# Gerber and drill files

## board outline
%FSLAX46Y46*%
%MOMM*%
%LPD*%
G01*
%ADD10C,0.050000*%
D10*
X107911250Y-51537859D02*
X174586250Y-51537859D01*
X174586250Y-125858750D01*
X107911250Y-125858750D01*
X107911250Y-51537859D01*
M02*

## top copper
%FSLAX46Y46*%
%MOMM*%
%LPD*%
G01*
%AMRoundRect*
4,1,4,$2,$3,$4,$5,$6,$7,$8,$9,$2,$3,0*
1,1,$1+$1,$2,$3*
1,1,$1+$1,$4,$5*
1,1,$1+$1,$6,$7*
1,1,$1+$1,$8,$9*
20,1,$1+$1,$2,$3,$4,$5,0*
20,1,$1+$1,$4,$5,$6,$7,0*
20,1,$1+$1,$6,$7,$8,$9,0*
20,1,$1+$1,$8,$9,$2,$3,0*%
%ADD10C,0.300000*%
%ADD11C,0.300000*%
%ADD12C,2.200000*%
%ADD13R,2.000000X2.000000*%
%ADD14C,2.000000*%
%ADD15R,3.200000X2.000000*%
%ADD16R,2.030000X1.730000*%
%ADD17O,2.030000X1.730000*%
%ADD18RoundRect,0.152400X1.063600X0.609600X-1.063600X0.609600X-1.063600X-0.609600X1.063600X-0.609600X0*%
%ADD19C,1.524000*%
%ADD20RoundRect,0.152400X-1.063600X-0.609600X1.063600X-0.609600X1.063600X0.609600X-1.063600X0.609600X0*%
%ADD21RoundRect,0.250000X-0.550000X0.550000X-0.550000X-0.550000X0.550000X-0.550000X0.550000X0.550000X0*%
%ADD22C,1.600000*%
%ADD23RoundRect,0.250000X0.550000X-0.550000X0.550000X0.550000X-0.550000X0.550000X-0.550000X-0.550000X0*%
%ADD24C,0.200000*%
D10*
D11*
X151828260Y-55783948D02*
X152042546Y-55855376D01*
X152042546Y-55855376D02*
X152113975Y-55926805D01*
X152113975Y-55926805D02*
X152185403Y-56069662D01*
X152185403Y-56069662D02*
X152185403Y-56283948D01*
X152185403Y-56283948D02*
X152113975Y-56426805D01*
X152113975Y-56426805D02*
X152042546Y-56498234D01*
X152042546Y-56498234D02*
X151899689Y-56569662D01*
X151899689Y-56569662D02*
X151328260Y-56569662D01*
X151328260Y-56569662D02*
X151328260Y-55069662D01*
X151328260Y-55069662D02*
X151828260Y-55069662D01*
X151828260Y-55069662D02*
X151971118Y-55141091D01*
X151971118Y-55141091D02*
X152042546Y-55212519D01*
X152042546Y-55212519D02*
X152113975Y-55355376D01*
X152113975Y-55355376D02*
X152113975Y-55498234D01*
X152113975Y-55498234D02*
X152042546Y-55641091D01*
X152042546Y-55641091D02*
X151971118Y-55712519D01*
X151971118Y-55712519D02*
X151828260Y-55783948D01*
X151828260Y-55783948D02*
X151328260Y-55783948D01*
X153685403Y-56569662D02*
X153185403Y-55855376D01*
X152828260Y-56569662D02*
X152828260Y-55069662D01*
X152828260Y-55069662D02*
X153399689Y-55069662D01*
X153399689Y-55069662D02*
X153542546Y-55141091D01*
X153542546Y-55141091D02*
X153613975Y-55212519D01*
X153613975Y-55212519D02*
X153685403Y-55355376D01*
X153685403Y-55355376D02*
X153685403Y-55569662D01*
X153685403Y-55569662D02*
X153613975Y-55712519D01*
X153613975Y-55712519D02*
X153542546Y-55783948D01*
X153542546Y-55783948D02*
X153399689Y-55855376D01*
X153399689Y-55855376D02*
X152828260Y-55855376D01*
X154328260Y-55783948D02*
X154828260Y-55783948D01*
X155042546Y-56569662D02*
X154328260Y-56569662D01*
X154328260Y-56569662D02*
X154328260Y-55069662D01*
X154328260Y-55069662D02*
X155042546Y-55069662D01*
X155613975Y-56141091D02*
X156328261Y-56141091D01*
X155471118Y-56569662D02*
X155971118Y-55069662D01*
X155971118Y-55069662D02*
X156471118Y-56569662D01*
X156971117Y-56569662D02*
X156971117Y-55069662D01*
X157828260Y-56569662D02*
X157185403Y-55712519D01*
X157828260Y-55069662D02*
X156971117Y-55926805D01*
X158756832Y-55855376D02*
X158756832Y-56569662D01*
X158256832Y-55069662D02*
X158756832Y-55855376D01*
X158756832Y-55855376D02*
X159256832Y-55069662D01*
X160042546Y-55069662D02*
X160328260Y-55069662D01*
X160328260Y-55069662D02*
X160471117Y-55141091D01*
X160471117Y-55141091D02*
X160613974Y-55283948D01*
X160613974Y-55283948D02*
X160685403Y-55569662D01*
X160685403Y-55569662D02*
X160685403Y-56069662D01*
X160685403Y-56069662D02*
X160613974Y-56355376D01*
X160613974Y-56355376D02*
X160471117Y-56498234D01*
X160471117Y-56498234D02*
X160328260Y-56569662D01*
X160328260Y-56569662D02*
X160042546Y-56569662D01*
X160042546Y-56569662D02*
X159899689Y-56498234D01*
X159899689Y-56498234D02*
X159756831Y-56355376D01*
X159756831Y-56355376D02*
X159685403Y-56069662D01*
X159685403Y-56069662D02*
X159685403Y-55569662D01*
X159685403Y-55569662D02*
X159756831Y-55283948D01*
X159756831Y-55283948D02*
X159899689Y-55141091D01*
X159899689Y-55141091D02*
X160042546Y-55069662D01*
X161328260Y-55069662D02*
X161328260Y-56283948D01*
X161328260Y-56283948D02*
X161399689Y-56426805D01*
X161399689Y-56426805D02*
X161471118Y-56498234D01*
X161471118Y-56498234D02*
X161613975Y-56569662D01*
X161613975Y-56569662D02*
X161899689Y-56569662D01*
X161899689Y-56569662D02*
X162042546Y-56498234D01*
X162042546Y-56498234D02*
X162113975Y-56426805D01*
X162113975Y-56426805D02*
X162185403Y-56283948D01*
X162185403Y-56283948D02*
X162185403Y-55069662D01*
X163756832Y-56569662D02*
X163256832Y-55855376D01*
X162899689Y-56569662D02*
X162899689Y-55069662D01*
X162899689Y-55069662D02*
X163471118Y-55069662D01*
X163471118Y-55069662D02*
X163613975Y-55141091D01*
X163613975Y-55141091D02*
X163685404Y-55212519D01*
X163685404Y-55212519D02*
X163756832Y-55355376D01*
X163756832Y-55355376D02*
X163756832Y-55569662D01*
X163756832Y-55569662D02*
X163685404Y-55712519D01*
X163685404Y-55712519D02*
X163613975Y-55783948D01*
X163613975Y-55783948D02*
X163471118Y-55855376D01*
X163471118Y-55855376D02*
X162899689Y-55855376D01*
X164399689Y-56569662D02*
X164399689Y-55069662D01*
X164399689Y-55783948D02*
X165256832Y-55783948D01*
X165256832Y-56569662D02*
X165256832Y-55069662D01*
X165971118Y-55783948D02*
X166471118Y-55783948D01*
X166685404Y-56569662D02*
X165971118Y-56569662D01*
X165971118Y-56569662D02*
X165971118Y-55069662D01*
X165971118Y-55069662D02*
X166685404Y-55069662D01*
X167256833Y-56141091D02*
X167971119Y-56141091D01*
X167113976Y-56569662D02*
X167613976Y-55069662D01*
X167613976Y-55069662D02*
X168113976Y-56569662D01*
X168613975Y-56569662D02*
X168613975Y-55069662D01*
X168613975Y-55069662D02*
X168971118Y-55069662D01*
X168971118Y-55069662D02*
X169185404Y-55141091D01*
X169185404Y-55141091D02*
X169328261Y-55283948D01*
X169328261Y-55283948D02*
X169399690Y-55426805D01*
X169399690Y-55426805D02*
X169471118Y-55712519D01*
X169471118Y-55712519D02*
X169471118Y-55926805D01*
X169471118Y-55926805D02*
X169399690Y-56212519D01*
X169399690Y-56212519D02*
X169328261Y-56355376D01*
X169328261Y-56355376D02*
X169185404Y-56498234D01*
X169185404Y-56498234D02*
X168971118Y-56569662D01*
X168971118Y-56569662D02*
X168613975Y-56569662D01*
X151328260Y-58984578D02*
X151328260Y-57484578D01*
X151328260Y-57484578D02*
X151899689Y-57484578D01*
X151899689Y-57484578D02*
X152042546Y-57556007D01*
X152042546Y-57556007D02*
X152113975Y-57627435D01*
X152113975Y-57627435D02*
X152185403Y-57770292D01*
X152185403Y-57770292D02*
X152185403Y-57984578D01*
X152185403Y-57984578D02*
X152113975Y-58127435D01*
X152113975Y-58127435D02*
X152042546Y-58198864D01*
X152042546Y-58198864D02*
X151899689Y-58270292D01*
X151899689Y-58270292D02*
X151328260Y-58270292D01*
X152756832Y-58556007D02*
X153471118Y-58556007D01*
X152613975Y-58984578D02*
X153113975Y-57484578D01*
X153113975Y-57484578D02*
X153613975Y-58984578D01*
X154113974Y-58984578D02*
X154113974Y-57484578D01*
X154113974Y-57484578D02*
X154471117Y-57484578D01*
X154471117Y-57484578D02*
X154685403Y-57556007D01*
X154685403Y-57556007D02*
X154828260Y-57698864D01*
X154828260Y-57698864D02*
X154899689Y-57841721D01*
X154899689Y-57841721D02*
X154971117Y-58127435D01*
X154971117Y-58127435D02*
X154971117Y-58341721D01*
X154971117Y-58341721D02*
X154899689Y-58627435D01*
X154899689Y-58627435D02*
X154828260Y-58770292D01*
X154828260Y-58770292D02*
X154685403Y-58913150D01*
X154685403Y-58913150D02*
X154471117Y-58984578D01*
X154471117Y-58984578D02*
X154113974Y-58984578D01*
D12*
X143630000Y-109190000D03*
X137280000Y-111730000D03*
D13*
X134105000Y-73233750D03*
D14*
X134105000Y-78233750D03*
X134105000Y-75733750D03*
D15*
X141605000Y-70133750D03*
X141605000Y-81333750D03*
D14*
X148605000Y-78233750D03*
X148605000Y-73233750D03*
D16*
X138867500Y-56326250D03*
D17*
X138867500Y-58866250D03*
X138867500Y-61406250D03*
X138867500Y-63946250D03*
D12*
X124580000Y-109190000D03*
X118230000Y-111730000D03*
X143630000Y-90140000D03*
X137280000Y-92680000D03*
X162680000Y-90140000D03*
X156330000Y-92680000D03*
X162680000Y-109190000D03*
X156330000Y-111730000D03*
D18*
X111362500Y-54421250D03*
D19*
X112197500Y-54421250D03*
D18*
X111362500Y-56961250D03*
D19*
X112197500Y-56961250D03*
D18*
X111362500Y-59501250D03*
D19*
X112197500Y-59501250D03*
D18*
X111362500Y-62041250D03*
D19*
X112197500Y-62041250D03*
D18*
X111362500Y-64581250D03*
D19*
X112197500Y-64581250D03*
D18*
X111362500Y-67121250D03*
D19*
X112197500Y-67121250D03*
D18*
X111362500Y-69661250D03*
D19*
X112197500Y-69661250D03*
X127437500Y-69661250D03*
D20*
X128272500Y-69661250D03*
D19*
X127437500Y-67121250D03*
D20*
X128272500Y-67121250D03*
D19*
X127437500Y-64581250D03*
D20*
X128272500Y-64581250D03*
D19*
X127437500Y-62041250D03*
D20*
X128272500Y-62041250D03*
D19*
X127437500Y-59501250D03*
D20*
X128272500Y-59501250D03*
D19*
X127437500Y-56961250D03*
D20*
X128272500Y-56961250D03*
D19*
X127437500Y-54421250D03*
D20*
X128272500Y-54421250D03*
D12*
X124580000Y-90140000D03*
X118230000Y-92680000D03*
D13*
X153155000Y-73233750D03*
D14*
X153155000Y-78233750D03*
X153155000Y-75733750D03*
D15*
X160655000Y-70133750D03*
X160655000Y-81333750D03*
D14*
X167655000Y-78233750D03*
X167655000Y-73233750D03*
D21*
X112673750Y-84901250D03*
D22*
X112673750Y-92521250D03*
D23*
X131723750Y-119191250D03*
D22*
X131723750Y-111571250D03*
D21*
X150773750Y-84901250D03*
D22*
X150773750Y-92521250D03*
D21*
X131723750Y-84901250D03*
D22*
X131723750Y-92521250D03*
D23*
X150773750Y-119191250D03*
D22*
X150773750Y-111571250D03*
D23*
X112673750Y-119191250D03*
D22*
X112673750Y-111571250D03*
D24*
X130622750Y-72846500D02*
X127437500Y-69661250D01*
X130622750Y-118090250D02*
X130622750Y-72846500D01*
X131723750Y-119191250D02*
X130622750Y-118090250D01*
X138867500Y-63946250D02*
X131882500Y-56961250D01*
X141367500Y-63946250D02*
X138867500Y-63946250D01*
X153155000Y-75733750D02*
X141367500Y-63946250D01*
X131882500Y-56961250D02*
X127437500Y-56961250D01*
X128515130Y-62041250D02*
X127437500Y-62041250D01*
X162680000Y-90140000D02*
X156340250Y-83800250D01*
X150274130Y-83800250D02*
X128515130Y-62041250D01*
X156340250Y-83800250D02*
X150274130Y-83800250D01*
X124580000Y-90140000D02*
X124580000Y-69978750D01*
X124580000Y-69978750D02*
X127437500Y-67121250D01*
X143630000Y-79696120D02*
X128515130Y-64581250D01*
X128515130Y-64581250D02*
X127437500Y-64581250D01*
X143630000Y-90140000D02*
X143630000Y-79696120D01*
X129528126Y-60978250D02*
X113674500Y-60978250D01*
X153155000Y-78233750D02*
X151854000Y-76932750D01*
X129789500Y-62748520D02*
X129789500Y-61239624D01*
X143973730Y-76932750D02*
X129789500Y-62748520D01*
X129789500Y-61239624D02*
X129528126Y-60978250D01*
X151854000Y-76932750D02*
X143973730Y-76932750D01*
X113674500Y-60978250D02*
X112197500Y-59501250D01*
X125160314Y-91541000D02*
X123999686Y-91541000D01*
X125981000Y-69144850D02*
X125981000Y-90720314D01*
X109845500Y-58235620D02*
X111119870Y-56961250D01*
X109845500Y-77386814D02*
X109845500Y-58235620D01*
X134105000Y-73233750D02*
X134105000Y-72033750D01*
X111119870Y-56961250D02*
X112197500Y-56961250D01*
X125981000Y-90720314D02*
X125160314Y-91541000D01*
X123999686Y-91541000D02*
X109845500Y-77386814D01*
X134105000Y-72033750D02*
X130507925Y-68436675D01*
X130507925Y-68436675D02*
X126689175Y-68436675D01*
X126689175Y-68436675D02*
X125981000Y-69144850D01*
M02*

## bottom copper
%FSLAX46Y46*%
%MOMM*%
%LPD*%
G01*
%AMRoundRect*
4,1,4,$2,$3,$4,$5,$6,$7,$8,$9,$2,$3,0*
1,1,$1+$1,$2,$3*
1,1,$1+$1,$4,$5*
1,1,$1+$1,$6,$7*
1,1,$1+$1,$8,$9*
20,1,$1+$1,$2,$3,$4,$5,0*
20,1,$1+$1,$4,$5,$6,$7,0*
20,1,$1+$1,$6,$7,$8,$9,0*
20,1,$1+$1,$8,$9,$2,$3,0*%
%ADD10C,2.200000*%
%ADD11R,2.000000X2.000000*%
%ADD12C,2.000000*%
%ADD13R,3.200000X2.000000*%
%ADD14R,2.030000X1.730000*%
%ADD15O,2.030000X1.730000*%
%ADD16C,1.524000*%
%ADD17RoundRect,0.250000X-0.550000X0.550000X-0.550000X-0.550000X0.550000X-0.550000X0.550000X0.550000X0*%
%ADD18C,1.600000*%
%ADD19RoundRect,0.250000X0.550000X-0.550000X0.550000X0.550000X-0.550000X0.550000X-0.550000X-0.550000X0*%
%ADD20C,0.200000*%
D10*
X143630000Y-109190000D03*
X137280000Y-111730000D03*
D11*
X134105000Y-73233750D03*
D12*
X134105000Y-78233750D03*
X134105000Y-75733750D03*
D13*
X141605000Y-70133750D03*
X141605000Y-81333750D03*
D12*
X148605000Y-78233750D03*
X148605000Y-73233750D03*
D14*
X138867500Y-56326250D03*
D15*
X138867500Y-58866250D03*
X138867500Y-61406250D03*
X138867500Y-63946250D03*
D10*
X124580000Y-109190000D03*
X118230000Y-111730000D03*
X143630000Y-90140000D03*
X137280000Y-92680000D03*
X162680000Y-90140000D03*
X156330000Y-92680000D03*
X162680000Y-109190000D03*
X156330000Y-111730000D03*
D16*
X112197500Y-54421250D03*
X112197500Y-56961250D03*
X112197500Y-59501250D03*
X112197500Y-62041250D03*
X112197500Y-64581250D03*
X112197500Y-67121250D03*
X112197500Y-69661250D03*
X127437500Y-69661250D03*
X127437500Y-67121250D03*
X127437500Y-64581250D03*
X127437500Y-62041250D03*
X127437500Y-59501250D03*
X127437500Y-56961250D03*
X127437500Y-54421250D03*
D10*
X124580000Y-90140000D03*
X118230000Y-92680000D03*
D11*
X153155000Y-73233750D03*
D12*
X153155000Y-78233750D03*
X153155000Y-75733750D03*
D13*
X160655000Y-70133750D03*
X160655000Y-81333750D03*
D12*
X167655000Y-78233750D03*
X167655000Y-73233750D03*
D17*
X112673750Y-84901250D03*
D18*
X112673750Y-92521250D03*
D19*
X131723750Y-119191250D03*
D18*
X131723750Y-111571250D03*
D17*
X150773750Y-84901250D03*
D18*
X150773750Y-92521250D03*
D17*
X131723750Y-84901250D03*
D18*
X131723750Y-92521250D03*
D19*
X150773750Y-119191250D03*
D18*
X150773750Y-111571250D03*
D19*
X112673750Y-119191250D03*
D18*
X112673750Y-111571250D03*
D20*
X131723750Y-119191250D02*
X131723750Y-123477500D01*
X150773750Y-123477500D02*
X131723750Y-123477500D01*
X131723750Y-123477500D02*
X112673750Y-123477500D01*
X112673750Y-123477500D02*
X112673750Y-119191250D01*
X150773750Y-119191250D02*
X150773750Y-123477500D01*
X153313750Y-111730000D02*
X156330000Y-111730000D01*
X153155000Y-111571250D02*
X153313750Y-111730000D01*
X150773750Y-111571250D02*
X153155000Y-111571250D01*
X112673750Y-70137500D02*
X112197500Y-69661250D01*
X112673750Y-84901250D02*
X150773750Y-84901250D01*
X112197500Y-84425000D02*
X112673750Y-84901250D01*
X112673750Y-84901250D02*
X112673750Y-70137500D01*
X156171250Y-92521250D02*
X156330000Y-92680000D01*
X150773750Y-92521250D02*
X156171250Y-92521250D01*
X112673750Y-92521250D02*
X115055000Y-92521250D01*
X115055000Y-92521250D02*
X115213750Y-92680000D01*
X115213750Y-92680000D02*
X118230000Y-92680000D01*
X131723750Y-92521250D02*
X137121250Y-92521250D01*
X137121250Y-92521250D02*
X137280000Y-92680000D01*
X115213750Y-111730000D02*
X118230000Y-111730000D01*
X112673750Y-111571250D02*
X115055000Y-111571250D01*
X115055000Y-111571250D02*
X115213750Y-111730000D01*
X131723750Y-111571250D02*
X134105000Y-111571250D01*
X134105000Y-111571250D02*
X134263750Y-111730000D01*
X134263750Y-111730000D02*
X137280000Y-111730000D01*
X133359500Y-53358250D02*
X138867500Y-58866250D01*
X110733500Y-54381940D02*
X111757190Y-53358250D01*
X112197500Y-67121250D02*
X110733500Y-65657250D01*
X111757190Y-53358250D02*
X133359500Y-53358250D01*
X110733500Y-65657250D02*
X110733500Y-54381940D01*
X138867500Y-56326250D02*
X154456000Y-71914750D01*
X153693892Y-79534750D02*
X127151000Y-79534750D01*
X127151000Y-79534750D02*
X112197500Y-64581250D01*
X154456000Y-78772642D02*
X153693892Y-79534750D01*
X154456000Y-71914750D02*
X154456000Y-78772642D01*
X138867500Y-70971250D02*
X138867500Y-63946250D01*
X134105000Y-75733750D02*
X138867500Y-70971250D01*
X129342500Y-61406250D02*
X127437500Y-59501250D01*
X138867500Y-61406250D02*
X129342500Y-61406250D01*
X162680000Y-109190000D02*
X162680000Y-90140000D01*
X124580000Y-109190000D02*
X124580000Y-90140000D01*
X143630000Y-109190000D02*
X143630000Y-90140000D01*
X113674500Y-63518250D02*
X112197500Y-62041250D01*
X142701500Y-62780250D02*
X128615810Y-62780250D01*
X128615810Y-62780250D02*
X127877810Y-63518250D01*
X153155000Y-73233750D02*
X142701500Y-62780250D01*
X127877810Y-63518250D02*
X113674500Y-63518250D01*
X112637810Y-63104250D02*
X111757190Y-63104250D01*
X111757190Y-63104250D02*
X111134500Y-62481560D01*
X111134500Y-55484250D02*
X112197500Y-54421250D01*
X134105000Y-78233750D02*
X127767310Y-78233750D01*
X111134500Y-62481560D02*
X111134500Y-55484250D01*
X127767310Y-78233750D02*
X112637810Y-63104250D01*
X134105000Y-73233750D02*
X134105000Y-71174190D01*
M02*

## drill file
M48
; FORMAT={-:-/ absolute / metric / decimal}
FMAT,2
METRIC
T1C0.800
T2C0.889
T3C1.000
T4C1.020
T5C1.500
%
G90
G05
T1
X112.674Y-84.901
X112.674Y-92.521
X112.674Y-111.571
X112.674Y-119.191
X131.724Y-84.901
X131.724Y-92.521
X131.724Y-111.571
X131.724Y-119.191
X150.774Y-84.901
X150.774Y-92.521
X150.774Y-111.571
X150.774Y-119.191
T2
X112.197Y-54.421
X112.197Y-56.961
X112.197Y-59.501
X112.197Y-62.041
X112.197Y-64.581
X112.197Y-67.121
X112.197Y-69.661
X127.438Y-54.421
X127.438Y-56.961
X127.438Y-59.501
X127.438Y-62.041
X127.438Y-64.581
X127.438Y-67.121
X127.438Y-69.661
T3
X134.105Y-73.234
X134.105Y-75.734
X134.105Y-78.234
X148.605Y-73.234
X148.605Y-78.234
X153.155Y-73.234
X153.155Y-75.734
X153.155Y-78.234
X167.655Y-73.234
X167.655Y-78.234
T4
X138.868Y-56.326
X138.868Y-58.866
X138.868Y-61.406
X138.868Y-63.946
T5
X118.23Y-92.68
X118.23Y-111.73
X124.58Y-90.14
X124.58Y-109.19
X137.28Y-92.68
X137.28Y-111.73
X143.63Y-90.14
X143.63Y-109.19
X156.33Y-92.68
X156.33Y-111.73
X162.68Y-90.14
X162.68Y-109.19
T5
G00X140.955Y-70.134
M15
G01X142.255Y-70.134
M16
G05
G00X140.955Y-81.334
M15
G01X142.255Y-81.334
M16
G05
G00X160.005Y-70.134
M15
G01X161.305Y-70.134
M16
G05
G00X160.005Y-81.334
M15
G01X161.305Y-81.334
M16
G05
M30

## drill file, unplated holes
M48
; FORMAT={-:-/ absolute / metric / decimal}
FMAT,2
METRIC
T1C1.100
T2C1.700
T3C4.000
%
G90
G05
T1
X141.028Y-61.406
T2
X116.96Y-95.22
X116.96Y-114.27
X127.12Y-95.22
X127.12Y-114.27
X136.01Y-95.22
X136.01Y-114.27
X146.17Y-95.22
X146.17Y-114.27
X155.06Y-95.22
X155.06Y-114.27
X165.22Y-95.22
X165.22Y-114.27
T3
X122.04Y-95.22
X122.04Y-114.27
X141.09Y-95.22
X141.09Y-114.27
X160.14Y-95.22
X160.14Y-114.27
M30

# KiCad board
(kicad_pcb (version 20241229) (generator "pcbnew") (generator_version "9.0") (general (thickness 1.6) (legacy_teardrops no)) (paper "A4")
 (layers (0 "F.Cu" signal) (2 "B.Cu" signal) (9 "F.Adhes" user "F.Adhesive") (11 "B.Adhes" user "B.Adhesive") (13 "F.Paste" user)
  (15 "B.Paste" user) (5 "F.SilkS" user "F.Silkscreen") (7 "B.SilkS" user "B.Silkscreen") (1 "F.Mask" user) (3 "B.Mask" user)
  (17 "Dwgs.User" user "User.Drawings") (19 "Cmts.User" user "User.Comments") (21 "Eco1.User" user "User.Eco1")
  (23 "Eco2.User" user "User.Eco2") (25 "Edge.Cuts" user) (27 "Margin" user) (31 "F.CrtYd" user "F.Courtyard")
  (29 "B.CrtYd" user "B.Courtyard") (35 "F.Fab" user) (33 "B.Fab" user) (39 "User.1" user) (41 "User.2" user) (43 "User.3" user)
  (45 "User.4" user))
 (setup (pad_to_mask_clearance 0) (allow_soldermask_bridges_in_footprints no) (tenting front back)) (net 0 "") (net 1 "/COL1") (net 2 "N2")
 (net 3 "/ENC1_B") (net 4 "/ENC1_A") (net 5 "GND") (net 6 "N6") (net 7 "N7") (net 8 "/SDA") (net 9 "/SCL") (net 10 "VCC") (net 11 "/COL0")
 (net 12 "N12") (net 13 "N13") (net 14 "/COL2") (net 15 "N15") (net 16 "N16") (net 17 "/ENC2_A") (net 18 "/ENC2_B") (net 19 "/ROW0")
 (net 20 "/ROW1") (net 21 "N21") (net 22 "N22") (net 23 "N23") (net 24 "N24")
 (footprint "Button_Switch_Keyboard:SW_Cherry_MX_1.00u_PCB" (layer "F.Cu") (at 143.63 109.19)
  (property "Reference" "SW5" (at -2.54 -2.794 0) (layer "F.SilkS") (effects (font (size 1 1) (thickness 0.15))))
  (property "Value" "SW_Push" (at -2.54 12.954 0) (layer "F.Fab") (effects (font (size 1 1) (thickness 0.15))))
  (pad "" np_thru_hole circle (at -7.62 5.08) (size 1.7 1.7) (drill 1.7) (layers "*.Cu" "*.Mask"))
  (pad "" np_thru_hole circle (at -2.54 5.08) (size 4 4) (drill 4) (layers "*.Cu" "*.Mask"))
  (pad "" np_thru_hole circle (at 2.54 5.08) (size 1.7 1.7) (drill 1.7) (layers "*.Cu" "*.Mask"))
  (pad "1" thru_hole circle (at 0 0) (size 2.2 2.2) (drill 1.5) (layers "*.Cu" "*.Mask") (remove_unused_layers no) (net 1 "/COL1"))
  (pad "2" thru_hole circle (at -6.35 2.54) (size 2.2 2.2) (drill 1.5) (layers "*.Cu" "*.Mask") (remove_unused_layers no) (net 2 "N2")))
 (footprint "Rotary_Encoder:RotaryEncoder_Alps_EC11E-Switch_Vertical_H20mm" (layer "F.Cu") (at 134.105 73.23375)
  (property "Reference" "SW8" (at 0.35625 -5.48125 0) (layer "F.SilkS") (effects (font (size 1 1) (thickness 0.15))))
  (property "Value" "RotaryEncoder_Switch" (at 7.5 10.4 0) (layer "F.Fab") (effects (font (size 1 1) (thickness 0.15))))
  (pad "A" thru_hole rect (at 0 0) (size 2 2) (drill 1) (layers "*.Cu" "*.Mask") (remove_unused_layers no) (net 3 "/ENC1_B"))
  (pad "B" thru_hole circle (at 0 5) (size 2 2) (drill 1) (layers "*.Cu" "*.Mask") (remove_unused_layers no) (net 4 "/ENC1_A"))
  (pad "C" thru_hole circle (at 0 2.5) (size 2 2) (drill 1) (layers "*.Cu" "*.Mask") (remove_unused_layers no) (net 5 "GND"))
  (pad "MP" thru_hole rect (at 7.5 -3.1) (size 3.2 2) (drill oval 2.8 1.5) (layers "*.Cu" "*.Mask") (remove_unused_layers no))
  (pad "MP" thru_hole rect (at 7.5 8.1) (size 3.2 2) (drill oval 2.8 1.5) (layers "*.Cu" "*.Mask") (remove_unused_layers no))
  (pad "S1" thru_hole circle (at 14.5 5) (size 2 2) (drill 1) (layers "*.Cu" "*.Mask") (remove_unused_layers no) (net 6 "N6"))
  (pad "S2" thru_hole circle (at 14.5 0) (size 2 2) (drill 1) (layers "*.Cu" "*.Mask") (remove_unused_layers no) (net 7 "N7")))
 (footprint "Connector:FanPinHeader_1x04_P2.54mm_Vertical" (layer "F.Cu") (at 138.8675 56.32625 -90)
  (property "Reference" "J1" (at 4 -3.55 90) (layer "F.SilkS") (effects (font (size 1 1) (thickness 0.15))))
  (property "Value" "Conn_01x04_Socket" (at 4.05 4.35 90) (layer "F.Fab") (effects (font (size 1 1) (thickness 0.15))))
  (pad "" np_thru_hole circle (at 5.08 -2.16) (size 1.1 1.1) (drill 1.1) (layers "*.Cu" "*.Mask"))
  (pad "1" thru_hole rect (at 0 0) (size 2.03 1.73) (drill 1.02) (layers "*.Cu" "*.Mask") (remove_unused_layers no) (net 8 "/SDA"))
  (pad "2" thru_hole oval (at 2.54 0) (size 2.03 1.73) (drill 1.02) (layers "*.Cu" "*.Mask") (remove_unused_layers no) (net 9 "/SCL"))
  (pad "3" thru_hole oval (at 5.08 0) (size 2.03 1.73) (drill 1.02) (layers "*.Cu" "*.Mask") (remove_unused_layers no) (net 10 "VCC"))
  (pad "4" thru_hole oval (at 7.62 0) (size 2.03 1.73) (drill 1.02) (layers "*.Cu" "*.Mask") (remove_unused_layers no) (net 5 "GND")))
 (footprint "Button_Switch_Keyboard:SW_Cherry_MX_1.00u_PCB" (layer "F.Cu") (at 124.58 109.19)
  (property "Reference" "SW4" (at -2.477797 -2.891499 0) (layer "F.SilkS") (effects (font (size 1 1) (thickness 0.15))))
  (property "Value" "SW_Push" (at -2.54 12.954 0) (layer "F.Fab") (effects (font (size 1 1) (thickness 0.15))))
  (pad "" np_thru_hole circle (at -7.62 5.08) (size 1.7 1.7) (drill 1.7) (layers "*.Cu" "*.Mask"))
  (pad "" np_thru_hole circle (at -2.54 5.08) (size 4 4) (drill 4) (layers "*.Cu" "*.Mask"))
  (pad "" np_thru_hole circle (at 2.54 5.08) (size 1.7 1.7) (drill 1.7) (layers "*.Cu" "*.Mask"))
  (pad "1" thru_hole circle (at 0 0) (size 2.2 2.2) (drill 1.5) (layers "*.Cu" "*.Mask") (remove_unused_layers no) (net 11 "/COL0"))
  (pad "2" thru_hole circle (at -6.35 2.54) (size 2.2 2.2) (drill 1.5) (layers "*.Cu" "*.Mask") (remove_unused_layers no) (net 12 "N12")))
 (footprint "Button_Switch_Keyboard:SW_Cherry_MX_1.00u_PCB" (layer "F.Cu") (at 143.63 90.14)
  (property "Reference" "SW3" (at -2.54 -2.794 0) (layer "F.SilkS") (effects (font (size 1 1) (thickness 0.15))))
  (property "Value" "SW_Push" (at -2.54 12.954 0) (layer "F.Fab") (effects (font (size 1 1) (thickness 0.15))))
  (pad "" np_thru_hole circle (at -7.62 5.08) (size 1.7 1.7) (drill 1.7) (layers "*.Cu" "*.Mask"))
  (pad "" np_thru_hole circle (at -2.54 5.08) (size 4 4) (drill 4) (layers "*.Cu" "*.Mask"))
  (pad "" np_thru_hole circle (at 2.54 5.08) (size 1.7 1.7) (drill 1.7) (layers "*.Cu" "*.Mask"))
  (pad "1" thru_hole circle (at 0 0) (size 2.2 2.2) (drill 1.5) (layers "*.Cu" "*.Mask") (remove_unused_layers no) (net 1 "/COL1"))
  (pad "2" thru_hole circle (at -6.35 2.54) (size 2.2 2.2) (drill 1.5) (layers "*.Cu" "*.Mask") (remove_unused_layers no) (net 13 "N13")))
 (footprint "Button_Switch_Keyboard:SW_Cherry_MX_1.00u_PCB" (layer "F.Cu") (at 162.68 90.14)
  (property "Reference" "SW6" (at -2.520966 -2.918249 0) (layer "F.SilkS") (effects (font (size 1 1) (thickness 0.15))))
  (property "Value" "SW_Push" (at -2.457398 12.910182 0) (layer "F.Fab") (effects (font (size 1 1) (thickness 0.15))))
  (pad "" np_thru_hole circle (at -7.62 5.08) (size 1.7 1.7) (drill 1.7) (layers "*.Cu" "*.Mask"))
  (pad "" np_thru_hole circle (at -2.54 5.08) (size 4 4) (drill 4) (layers "*.Cu" "*.Mask"))
  (pad "" np_thru_hole circle (at 2.54 5.08) (size 1.7 1.7) (drill 1.7) (layers "*.Cu" "*.Mask"))
  (pad "1" thru_hole circle (at 0 0) (size 2.2 2.2) (drill 1.5) (layers "*.Cu" "*.Mask") (remove_unused_layers no) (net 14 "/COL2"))
  (pad "2" thru_hole circle (at -6.35 2.54) (size 2.2 2.2) (drill 1.5) (layers "*.Cu" "*.Mask") (remove_unused_layers no) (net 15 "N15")))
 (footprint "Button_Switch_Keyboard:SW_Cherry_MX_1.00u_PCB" (layer "F.Cu") (at 162.68 109.19)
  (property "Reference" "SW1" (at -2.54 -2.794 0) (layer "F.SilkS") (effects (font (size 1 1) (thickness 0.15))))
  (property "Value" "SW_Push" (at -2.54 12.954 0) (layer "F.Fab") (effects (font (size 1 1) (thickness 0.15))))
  (pad "" np_thru_hole circle (at -7.62 5.08) (size 1.7 1.7) (drill 1.7) (layers "*.Cu" "*.Mask"))
  (pad "" np_thru_hole circle (at -2.54 5.08) (size 4 4) (drill 4) (layers "*.Cu" "*.Mask"))
  (pad "" np_thru_hole circle (at 2.54 5.08) (size 1.7 1.7) (drill 1.7) (layers "*.Cu" "*.Mask"))
  (pad "1" thru_hole circle (at 0 0) (size 2.2 2.2) (drill 1.5) (layers "*.Cu" "*.Mask") (remove_unused_layers no) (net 14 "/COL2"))
  (pad "2" thru_hole circle (at -6.35 2.54) (size 2.2 2.2) (drill 1.5) (layers "*.Cu" "*.Mask") (remove_unused_layers no) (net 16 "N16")))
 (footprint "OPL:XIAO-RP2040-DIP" (layer "F.Cu") (at 119.8175 62.04125)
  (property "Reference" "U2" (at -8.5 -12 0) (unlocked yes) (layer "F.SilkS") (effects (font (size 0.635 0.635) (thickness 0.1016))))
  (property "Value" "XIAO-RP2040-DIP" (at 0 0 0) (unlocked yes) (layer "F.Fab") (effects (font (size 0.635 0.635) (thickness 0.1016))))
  (pad "1" smd roundrect (at -8.455 -7.62 180) (size 2.432 1.524) (layers "F.Cu" "F.Mask") (roundrect_rratio 0.1) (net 4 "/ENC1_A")
   (thermal_bridge_angle 45))
  (pad "1" thru_hole circle (at -7.62 -7.62 180) (size 1.524 1.524) (drill 0.889) (layers "*.Cu" "*.Mask") (remove_unused_layers no)
   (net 4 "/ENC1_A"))
  (pad "2" smd roundrect (at -8.455 -5.08 180) (size 2.432 1.524) (layers "F.Cu" "F.Mask") (roundrect_rratio 0.1) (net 3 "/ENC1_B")
   (thermal_bridge_angle 45))
  (pad "2" thru_hole circle (at -7.62 -5.08 180) (size 1.524 1.524) (drill 0.889) (layers "*.Cu" "*.Mask") (remove_unused_layers no)
   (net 3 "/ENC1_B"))
  (pad "3" smd roundrect (at -8.455 -2.54 180) (size 2.432 1.524) (layers "F.Cu" "F.Mask") (roundrect_rratio 0.1) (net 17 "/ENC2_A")
   (thermal_bridge_angle 45))
  (pad "3" thru_hole circle (at -7.62 -2.54 180) (size 1.524 1.524) (drill 0.889) (layers "*.Cu" "*.Mask") (remove_unused_layers no)
   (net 17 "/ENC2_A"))
  (pad "4" smd roundrect (at -8.455 0 180) (size 2.432 1.524) (layers "F.Cu" "F.Mask") (roundrect_rratio 0.1) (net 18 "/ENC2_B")
   (thermal_bridge_angle 45))
  (pad "4" thru_hole circle (at -7.62 0 180) (size 1.524 1.524) (drill 0.889) (layers "*.Cu" "*.Mask") (remove_unused_layers no)
   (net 18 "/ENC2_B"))
  (pad "5" smd roundrect (at -8.455 2.54 180) (size 2.432 1.524) (layers "F.Cu" "F.Mask") (roundrect_rratio 0.1) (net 8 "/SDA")
   (thermal_bridge_angle 45))
  (pad "5" thru_hole circle (at -7.62 2.54 180) (size 1.524 1.524) (drill 0.889) (layers "*.Cu" "*.Mask") (remove_unused_layers no)
   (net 8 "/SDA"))
  (pad "6" smd roundrect (at -8.455 5.08 180) (size 2.432 1.524) (layers "F.Cu" "F.Mask") (roundrect_rratio 0.1) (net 9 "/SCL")
   (thermal_bridge_angle 45))
  (pad "6" thru_hole circle (at -7.62 5.08 180) (size 1.524 1.524) (drill 0.889) (layers "*.Cu" "*.Mask") (remove_unused_layers no)
   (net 9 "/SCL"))
  (pad "7" smd roundrect (at -8.455 7.62 180) (size 2.432 1.524) (layers "F.Cu" "F.Mask") (roundrect_rratio 0.1) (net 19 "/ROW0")
   (thermal_bridge_angle 45))
  (pad "7" thru_hole circle (at -7.62 7.62 180) (size 1.524 1.524) (drill 0.889) (layers "*.Cu" "*.Mask") (remove_unused_layers no)
   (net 19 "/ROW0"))
  (pad "8" thru_hole circle (at 7.62 7.62) (size 1.524 1.524) (drill 0.889) (layers "*.Cu" "*.Mask") (remove_unused_layers no)
   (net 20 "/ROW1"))
  (pad "8" smd roundrect (at 8.455 7.62) (size 2.432 1.524) (layers "F.Cu" "F.Mask") (roundrect_rratio 0.1) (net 20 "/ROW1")
   (thermal_bridge_angle 45))
  (pad "9" thru_hole circle (at 7.62 5.08) (size 1.524 1.524) (drill 0.889) (layers "*.Cu" "*.Mask") (remove_unused_layers no)
   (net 11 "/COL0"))
  (pad "9" smd roundrect (at 8.455 5.08) (size 2.432 1.524) (layers "F.Cu" "F.Mask") (roundrect_rratio 0.1) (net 11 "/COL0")
   (thermal_bridge_angle 45))
  (pad "10" thru_hole circle (at 7.62 2.54) (size 1.524 1.524) (drill 0.889) (layers "*.Cu" "*.Mask") (remove_unused_layers no)
   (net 1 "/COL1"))
  (pad "10" smd roundrect (at 8.455 2.54) (size 2.432 1.524) (layers "F.Cu" "F.Mask") (roundrect_rratio 0.1) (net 1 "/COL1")
   (thermal_bridge_angle 45))
  (pad "11" thru_hole circle (at 7.62 0) (size 1.524 1.524) (drill 0.889) (layers "*.Cu" "*.Mask") (remove_unused_layers no)
   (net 14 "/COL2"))
  (pad "11" smd roundrect (at 8.455 0) (size 2.432 1.524) (layers "F.Cu" "F.Mask") (roundrect_rratio 0.1) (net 14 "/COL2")
   (thermal_bridge_angle 45))
  (pad "12" thru_hole circle (at 7.62 -2.54) (size 1.524 1.524) (drill 0.889) (layers "*.Cu" "*.Mask") (remove_unused_layers no)
   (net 10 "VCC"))
  (pad "12" smd roundrect (at 8.455 -2.54) (size 2.432 1.524) (layers "F.Cu" "F.Mask") (roundrect_rratio 0.1) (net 10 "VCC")
   (thermal_bridge_angle 45))
  (pad "13" thru_hole circle (at 7.62 -5.08) (size 1.524 1.524) (drill 0.889) (layers "*.Cu" "*.Mask") (remove_unused_layers no)
   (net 5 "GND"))
  (pad "13" smd roundrect (at 8.455 -5.08) (size 2.432 1.524) (layers "F.Cu" "F.Mask") (roundrect_rratio 0.1) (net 5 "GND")
   (thermal_bridge_angle 45))
  (pad "14" thru_hole circle (at 7.62 -7.62) (size 1.524 1.524) (drill 0.889) (layers "*.Cu" "*.Mask") (remove_unused_layers no)
   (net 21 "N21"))
  (pad "14" smd roundrect (at 8.455 -7.62) (size 2.432 1.524) (layers "F.Cu" "F.Mask") (roundrect_rratio 0.1) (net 21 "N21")
   (thermal_bridge_angle 45)))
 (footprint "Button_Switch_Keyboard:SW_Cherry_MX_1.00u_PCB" (layer "F.Cu") (at 124.58 90.14)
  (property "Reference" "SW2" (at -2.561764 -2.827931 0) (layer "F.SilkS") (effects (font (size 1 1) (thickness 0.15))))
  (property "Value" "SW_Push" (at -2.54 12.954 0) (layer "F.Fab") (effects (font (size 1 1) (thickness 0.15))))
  (pad "" np_thru_hole circle (at -7.62 5.08) (size 1.7 1.7) (drill 1.7) (layers "*.Cu" "*.Mask"))
  (pad "" np_thru_hole circle (at -2.54 5.08) (size 4 4) (drill 4) (layers "*.Cu" "*.Mask"))
  (pad "" np_thru_hole circle (at 2.54 5.08) (size 1.7 1.7) (drill 1.7) (layers "*.Cu" "*.Mask"))
  (pad "1" thru_hole circle (at 0 0) (size 2.2 2.2) (drill 1.5) (layers "*.Cu" "*.Mask") (remove_unused_layers no) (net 11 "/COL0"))
  (pad "2" thru_hole circle (at -6.35 2.54) (size 2.2 2.2) (drill 1.5) (layers "*.Cu" "*.Mask") (remove_unused_layers no) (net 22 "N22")))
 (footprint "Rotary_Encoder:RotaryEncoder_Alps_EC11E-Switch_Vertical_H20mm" (layer "F.Cu") (at 153.155 73.23375)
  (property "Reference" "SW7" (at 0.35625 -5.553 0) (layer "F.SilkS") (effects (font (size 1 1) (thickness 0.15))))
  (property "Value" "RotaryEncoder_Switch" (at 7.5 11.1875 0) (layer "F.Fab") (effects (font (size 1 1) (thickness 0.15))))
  (pad "A" thru_hole rect (at 0 0) (size 2 2) (drill 1) (layers "*.Cu" "*.Mask") (remove_unused_layers no) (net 18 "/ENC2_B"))
  (pad "B" thru_hole circle (at 0 5) (size 2 2) (drill 1) (layers "*.Cu" "*.Mask") (remove_unused_layers no) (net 17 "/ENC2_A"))
  (pad "C" thru_hole circle (at 0 2.5) (size 2 2) (drill 1) (layers "*.Cu" "*.Mask") (remove_unused_layers no) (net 5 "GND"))
  (pad "MP" thru_hole rect (at 7.5 -3.1) (size 3.2 2) (drill oval 2.8 1.5) (layers "*.Cu" "*.Mask") (remove_unused_layers no))
  (pad "MP" thru_hole rect (at 7.5 8.1) (size 3.2 2) (drill oval 2.8 1.5) (layers "*.Cu" "*.Mask") (remove_unused_layers no))
  (pad "S1" thru_hole circle (at 14.5 5) (size 2 2) (drill 1) (layers "*.Cu" "*.Mask") (remove_unused_layers no) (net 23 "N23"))
  (pad "S2" thru_hole circle (at 14.5 0) (size 2 2) (drill 1) (layers "*.Cu" "*.Mask") (remove_unused_layers no) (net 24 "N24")))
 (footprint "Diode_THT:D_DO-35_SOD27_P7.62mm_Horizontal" (layer "B.Cu") (at 112.67375 84.90125 -90)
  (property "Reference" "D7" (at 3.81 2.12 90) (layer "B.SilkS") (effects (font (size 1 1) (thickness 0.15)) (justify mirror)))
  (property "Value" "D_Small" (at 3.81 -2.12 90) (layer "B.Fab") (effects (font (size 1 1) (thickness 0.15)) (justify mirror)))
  (pad "1" thru_hole roundrect (at 0 0 270) (size 1.6 1.6) (drill 0.8) (layers "*.Cu" "*.Mask") (remove_unused_layers no)
   (roundrect_rratio 0.15625) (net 19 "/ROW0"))
  (pad "2" thru_hole circle (at 7.62 0 270) (size 1.6 1.6) (drill 0.8) (layers "*.Cu" "*.Mask") (remove_unused_layers no) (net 22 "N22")))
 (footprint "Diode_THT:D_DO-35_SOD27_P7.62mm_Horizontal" (layer "B.Cu") (at 131.72375 119.19125 90)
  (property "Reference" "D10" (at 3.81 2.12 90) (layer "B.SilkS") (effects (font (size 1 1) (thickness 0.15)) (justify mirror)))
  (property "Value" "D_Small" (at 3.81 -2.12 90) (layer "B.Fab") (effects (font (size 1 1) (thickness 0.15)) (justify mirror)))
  (pad "1" thru_hole roundrect (at 0 0 90) (size 1.6 1.6) (drill 0.8) (layers "*.Cu" "*.Mask") (remove_unused_layers no)
   (roundrect_rratio 0.15625) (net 20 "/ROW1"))
  (pad "2" thru_hole circle (at 7.62 0 90) (size 1.6 1.6) (drill 0.8) (layers "*.Cu" "*.Mask") (remove_unused_layers no) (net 2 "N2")))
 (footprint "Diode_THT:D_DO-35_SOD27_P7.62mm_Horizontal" (layer "B.Cu") (at 150.77375 84.90125 -90)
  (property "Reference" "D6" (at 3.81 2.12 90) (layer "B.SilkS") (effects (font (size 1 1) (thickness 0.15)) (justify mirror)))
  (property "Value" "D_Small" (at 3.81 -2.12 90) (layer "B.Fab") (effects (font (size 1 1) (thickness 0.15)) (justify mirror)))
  (pad "1" thru_hole roundrect (at 0 0 270) (size 1.6 1.6) (drill 0.8) (layers "*.Cu" "*.Mask") (remove_unused_layers no)
   (roundrect_rratio 0.15625) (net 19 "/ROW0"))
  (pad "2" thru_hole circle (at 7.62 0 270) (size 1.6 1.6) (drill 0.8) (layers "*.Cu" "*.Mask") (remove_unused_layers no) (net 15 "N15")))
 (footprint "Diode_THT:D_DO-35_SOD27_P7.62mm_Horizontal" (layer "B.Cu") (at 131.72375 84.90125 -90)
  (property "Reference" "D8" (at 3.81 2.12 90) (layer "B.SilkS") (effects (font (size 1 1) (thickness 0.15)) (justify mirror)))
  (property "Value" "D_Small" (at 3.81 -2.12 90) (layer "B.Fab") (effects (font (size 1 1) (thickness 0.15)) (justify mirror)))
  (pad "1" thru_hole roundrect (at 0 0 270) (size 1.6 1.6) (drill 0.8) (layers "*.Cu" "*.Mask") (remove_unused_layers no)
   (roundrect_rratio 0.15625) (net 19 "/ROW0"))
  (pad "2" thru_hole circle (at 7.62 0 270) (size 1.6 1.6) (drill 0.8) (layers "*.Cu" "*.Mask") (remove_unused_layers no) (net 13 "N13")))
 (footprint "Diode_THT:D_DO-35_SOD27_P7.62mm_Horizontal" (layer "B.Cu") (at 150.77375 119.19125 90)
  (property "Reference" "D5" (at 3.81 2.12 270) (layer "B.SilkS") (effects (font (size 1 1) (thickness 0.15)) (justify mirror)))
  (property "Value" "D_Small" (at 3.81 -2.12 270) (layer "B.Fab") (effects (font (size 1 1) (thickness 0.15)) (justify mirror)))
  (pad "1" thru_hole roundrect (at 0 0 90) (size 1.6 1.6) (drill 0.8) (layers "*.Cu" "*.Mask") (remove_unused_layers no)
   (roundrect_rratio 0.15625) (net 20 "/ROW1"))
  (pad "2" thru_hole circle (at 7.62 0 90) (size 1.6 1.6) (drill 0.8) (layers "*.Cu" "*.Mask") (remove_unused_layers no) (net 16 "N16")))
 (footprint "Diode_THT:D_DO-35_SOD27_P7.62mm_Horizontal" (layer "B.Cu") (at 112.67375 119.19125 90)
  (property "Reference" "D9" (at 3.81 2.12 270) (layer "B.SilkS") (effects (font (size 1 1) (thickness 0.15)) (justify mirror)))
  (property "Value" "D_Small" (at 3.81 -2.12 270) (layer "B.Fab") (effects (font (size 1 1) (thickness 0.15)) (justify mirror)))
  (pad "1" thru_hole roundrect (at 0 0 90) (size 1.6 1.6) (drill 0.8) (layers "*.Cu" "*.Mask") (remove_unused_layers no)
   (roundrect_rratio 0.15625) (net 20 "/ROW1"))
  (pad "2" thru_hole circle (at 7.62 0 90) (size 1.6 1.6) (drill 0.8) (layers "*.Cu" "*.Mask") (remove_unused_layers no) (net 12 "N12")))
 (gr_rect (start 107.91125 51.537859) (end 174.58625 125.85875) (stroke (width 0.05) (type default)) (fill no) (layer "Edge.Cuts"))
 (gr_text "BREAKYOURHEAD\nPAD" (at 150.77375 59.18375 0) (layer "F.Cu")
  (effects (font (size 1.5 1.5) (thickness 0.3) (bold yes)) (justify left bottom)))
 (segment (start 130.62275 72.8465) (end 127.4375 69.66125) (width 0.2) (layer "F.Cu") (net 20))
 (segment (start 130.62275 118.09025) (end 130.62275 72.8465) (width 0.2) (layer "F.Cu") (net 20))
 (segment (start 131.72375 119.19125) (end 130.62275 118.09025) (width 0.2) (layer "F.Cu") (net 20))
 (segment (start 131.72375 119.19125) (end 131.72375 123.4775) (width 0.2) (layer "B.Cu") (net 20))
 (segment (start 150.77375 123.4775) (end 131.72375 123.4775) (width 0.2) (layer "B.Cu") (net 20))
 (segment (start 131.72375 123.4775) (end 112.67375 123.4775) (width 0.2) (layer "B.Cu") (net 20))
 (segment (start 112.67375 123.4775) (end 112.67375 119.19125) (width 0.2) (layer "B.Cu") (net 20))
 (segment (start 150.77375 119.19125) (end 150.77375 123.4775) (width 0.2) (layer "B.Cu") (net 20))
 (segment (start 153.31375 111.73) (end 156.33 111.73) (width 0.2) (layer "B.Cu") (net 16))
 (segment (start 153.155 111.57125) (end 153.31375 111.73) (width 0.2) (layer "B.Cu") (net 16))
 (segment (start 150.77375 111.57125) (end 153.155 111.57125) (width 0.2) (layer "B.Cu") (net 16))
 (segment (start 112.67375 70.1375) (end 112.1975 69.66125) (width 0.2) (layer "B.Cu") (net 19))
 (segment (start 112.67375 84.90125) (end 150.77375 84.90125) (width 0.2) (layer "B.Cu") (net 19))
 (segment (start 112.1975 84.425) (end 112.67375 84.90125) (width 0.2) (layer "B.Cu") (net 19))
 (segment (start 112.67375 84.90125) (end 112.67375 70.1375) (width 0.2) (layer "B.Cu") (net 19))
 (segment (start 156.17125 92.52125) (end 156.33 92.68) (width 0.2) (layer "B.Cu") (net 15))
 (segment (start 150.77375 92.52125) (end 156.17125 92.52125) (width 0.2) (layer "B.Cu") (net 15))
 (segment (start 112.67375 92.52125) (end 115.055 92.52125) (width 0.2) (layer "B.Cu") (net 22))
 (segment (start 115.055 92.52125) (end 115.21375 92.68) (width 0.2) (layer "B.Cu") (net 22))
 (segment (start 115.21375 92.68) (end 118.23 92.68) (width 0.2) (layer "B.Cu") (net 22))
 (segment (start 131.72375 92.52125) (end 137.12125 92.52125) (width 0.2) (layer "B.Cu") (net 13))
 (segment (start 137.12125 92.52125) (end 137.28 92.68) (width 0.2) (layer "B.Cu") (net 13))
 (segment (start 115.21375 111.73) (end 118.23 111.73) (width 0.2) (layer "B.Cu") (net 12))
 (segment (start 112.67375 111.57125) (end 115.055 111.57125) (width 0.2) (layer "B.Cu") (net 12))
 (segment (start 115.055 111.57125) (end 115.21375 111.73) (width 0.2) (layer "B.Cu") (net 12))
 (segment (start 131.72375 111.57125) (end 134.105 111.57125) (width 0.2) (layer "B.Cu") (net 2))
 (segment (start 134.105 111.57125) (end 134.26375 111.73) (width 0.2) (layer "B.Cu") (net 2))
 (segment (start 134.26375 111.73) (end 137.28 111.73) (width 0.2) (layer "B.Cu") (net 2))
 (segment (start 133.3595 53.35825) (end 138.8675 58.86625) (width 0.2) (layer "B.Cu") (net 9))
 (segment (start 110.7335 54.38194) (end 111.75719 53.35825) (width 0.2) (layer "B.Cu") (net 9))
 (segment (start 112.1975 67.12125) (end 110.7335 65.65725) (width 0.2) (layer "B.Cu") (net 9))
 (segment (start 111.75719 53.35825) (end 133.3595 53.35825) (width 0.2) (layer "B.Cu") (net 9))
 (segment (start 110.7335 65.65725) (end 110.7335 54.38194) (width 0.2) (layer "B.Cu") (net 9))
 (segment (start 138.8675 56.32625) (end 154.456 71.91475) (width 0.2) (layer "B.Cu") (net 8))
 (segment (start 153.693892 79.53475) (end 127.151 79.53475) (width 0.2) (layer "B.Cu") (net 8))
 (segment (start 127.151 79.53475) (end 112.1975 64.58125) (width 0.2) (layer "B.Cu") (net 8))
 (segment (start 154.456 78.772642) (end 153.693892 79.53475) (width 0.2) (layer "B.Cu") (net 8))
 (segment (start 154.456 71.91475) (end 154.456 78.772642) (width 0.2) (layer "B.Cu") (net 8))
 (segment (start 138.8675 63.94625) (end 131.8825 56.96125) (width 0.2) (layer "F.Cu") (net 5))
 (segment (start 141.3675 63.94625) (end 138.8675 63.94625) (width 0.2) (layer "F.Cu") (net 5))
 (segment (start 153.155 75.73375) (end 141.3675 63.94625) (width 0.2) (layer "F.Cu") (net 5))
 (segment (start 131.8825 56.96125) (end 127.4375 56.96125) (width 0.2) (layer "F.Cu") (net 5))
 (segment (start 138.8675 70.97125) (end 138.8675 63.94625) (width 0.2) (layer "B.Cu") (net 5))
 (segment (start 134.105 75.73375) (end 138.8675 70.97125) (width 0.2) (layer "B.Cu") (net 5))
 (segment (start 129.3425 61.40625) (end 127.4375 59.50125) (width 0.2) (layer "B.Cu") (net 10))
 (segment (start 138.8675 61.40625) (end 129.3425 61.40625) (width 0.2) (layer "B.Cu") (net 10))
 (segment (start 128.51513 62.04125) (end 127.4375 62.04125) (width 0.2) (layer "F.Cu") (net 14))
 (segment (start 162.68 90.14) (end 156.34025 83.80025) (width 0.2) (layer "F.Cu") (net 14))
 (segment (start 150.27413 83.80025) (end 128.51513 62.04125) (width 0.2) (layer "F.Cu") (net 14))
 (segment (start 156.34025 83.80025) (end 150.27413 83.80025) (width 0.2) (layer "F.Cu") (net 14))
 (segment (start 162.68 109.19) (end 162.68 90.14) (width 0.2) (layer "B.Cu") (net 14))
 (segment (start 124.58 90.14) (end 124.58 69.97875) (width 0.2) (layer "F.Cu") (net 11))
 (segment (start 124.58 69.97875) (end 127.4375 67.12125) (width 0.2) (layer "F.Cu") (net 11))
 (segment (start 124.58 109.19) (end 124.58 90.14) (width 0.2) (layer "B.Cu") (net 11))
 (segment (start 143.63 79.69612) (end 128.51513 64.58125) (width 0.2) (layer "F.Cu") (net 1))
 (segment (start 128.51513 64.58125) (end 127.4375 64.58125) (width 0.2) (layer "F.Cu") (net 1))
 (segment (start 143.63 90.14) (end 143.63 79.69612) (width 0.2) (layer "F.Cu") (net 1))
 (segment (start 143.63 109.19) (end 143.63 90.14) (width 0.2) (layer "B.Cu") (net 1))
 (segment (start 129.528126 60.97825) (end 113.6745 60.97825) (width 0.2) (layer "F.Cu") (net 17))
 (segment (start 153.155 78.23375) (end 151.854 76.93275) (width 0.2) (layer "F.Cu") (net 17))
 (segment (start 129.7895 62.74852) (end 129.7895 61.239624) (width 0.2) (layer "F.Cu") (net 17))
 (segment (start 143.97373 76.93275) (end 129.7895 62.74852) (width 0.2) (layer "F.Cu") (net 17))
 (segment (start 129.7895 61.239624) (end 129.528126 60.97825) (width 0.2) (layer "F.Cu") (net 17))
 (segment (start 151.854 76.93275) (end 143.97373 76.93275) (width 0.2) (layer "F.Cu") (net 17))
 (segment (start 113.6745 60.97825) (end 112.1975 59.50125) (width 0.2) (layer "F.Cu") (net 17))
 (segment (start 113.6745 63.51825) (end 112.1975 62.04125) (width 0.2) (layer "B.Cu") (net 18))
 (segment (start 142.7015 62.78025) (end 128.61581 62.78025) (width 0.2) (layer "B.Cu") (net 18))
 (segment (start 128.61581 62.78025) (end 127.87781 63.51825) (width 0.2) (layer "B.Cu") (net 18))
 (segment (start 153.155 73.23375) (end 142.7015 62.78025) (width 0.2) (layer "B.Cu") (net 18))
 (segment (start 127.87781 63.51825) (end 113.6745 63.51825) (width 0.2) (layer "B.Cu") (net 18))
 (segment (start 112.63781 63.10425) (end 111.75719 63.10425) (width 0.2) (layer "B.Cu") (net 4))
 (segment (start 111.75719 63.10425) (end 111.1345 62.48156) (width 0.2) (layer "B.Cu") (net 4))
 (segment (start 111.1345 55.48425) (end 112.1975 54.42125) (width 0.2) (layer "B.Cu") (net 4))
 (segment (start 134.105 78.23375) (end 127.76731 78.23375) (width 0.2) (layer "B.Cu") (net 4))
 (segment (start 111.1345 62.48156) (end 111.1345 55.48425) (width 0.2) (layer "B.Cu") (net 4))
 (segment (start 127.76731 78.23375) (end 112.63781 63.10425) (width 0.2) (layer "B.Cu") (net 4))
 (segment (start 125.160314 91.541) (end 123.999686 91.541) (width 0.2) (layer "F.Cu") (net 3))
 (segment (start 125.981 69.14485) (end 125.981 90.720314) (width 0.2) (layer "F.Cu") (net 3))
 (segment (start 109.8455 58.23562) (end 111.11987 56.96125) (width 0.2) (layer "F.Cu") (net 3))
 (segment (start 109.8455 77.386814) (end 109.8455 58.23562) (width 0.2) (layer "F.Cu") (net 3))
 (segment (start 134.105 73.23375) (end 134.105 72.03375) (width 0.2) (layer "F.Cu") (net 3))
 (segment (start 111.11987 56.96125) (end 112.1975 56.96125) (width 0.2) (layer "F.Cu") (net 3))
 (segment (start 125.981 90.720314) (end 125.160314 91.541) (width 0.2) (layer "F.Cu") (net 3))
 (segment (start 123.999686 91.541) (end 109.8455 77.386814) (width 0.2) (layer "F.Cu") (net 3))
 (segment (start 134.105 72.03375) (end 130.507925 68.436675) (width 0.2) (layer "F.Cu") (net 3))
 (segment (start 130.507925 68.436675) (end 126.689175 68.436675) (width 0.2) (layer "F.Cu") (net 3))
 (segment (start 126.689175 68.436675) (end 125.981 69.14485) (width 0.2) (layer "F.Cu") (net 3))
 (segment (start 134.105 73.23375) (end 134.105 71.17419) (width 0.2) (layer "B.Cu") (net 3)))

